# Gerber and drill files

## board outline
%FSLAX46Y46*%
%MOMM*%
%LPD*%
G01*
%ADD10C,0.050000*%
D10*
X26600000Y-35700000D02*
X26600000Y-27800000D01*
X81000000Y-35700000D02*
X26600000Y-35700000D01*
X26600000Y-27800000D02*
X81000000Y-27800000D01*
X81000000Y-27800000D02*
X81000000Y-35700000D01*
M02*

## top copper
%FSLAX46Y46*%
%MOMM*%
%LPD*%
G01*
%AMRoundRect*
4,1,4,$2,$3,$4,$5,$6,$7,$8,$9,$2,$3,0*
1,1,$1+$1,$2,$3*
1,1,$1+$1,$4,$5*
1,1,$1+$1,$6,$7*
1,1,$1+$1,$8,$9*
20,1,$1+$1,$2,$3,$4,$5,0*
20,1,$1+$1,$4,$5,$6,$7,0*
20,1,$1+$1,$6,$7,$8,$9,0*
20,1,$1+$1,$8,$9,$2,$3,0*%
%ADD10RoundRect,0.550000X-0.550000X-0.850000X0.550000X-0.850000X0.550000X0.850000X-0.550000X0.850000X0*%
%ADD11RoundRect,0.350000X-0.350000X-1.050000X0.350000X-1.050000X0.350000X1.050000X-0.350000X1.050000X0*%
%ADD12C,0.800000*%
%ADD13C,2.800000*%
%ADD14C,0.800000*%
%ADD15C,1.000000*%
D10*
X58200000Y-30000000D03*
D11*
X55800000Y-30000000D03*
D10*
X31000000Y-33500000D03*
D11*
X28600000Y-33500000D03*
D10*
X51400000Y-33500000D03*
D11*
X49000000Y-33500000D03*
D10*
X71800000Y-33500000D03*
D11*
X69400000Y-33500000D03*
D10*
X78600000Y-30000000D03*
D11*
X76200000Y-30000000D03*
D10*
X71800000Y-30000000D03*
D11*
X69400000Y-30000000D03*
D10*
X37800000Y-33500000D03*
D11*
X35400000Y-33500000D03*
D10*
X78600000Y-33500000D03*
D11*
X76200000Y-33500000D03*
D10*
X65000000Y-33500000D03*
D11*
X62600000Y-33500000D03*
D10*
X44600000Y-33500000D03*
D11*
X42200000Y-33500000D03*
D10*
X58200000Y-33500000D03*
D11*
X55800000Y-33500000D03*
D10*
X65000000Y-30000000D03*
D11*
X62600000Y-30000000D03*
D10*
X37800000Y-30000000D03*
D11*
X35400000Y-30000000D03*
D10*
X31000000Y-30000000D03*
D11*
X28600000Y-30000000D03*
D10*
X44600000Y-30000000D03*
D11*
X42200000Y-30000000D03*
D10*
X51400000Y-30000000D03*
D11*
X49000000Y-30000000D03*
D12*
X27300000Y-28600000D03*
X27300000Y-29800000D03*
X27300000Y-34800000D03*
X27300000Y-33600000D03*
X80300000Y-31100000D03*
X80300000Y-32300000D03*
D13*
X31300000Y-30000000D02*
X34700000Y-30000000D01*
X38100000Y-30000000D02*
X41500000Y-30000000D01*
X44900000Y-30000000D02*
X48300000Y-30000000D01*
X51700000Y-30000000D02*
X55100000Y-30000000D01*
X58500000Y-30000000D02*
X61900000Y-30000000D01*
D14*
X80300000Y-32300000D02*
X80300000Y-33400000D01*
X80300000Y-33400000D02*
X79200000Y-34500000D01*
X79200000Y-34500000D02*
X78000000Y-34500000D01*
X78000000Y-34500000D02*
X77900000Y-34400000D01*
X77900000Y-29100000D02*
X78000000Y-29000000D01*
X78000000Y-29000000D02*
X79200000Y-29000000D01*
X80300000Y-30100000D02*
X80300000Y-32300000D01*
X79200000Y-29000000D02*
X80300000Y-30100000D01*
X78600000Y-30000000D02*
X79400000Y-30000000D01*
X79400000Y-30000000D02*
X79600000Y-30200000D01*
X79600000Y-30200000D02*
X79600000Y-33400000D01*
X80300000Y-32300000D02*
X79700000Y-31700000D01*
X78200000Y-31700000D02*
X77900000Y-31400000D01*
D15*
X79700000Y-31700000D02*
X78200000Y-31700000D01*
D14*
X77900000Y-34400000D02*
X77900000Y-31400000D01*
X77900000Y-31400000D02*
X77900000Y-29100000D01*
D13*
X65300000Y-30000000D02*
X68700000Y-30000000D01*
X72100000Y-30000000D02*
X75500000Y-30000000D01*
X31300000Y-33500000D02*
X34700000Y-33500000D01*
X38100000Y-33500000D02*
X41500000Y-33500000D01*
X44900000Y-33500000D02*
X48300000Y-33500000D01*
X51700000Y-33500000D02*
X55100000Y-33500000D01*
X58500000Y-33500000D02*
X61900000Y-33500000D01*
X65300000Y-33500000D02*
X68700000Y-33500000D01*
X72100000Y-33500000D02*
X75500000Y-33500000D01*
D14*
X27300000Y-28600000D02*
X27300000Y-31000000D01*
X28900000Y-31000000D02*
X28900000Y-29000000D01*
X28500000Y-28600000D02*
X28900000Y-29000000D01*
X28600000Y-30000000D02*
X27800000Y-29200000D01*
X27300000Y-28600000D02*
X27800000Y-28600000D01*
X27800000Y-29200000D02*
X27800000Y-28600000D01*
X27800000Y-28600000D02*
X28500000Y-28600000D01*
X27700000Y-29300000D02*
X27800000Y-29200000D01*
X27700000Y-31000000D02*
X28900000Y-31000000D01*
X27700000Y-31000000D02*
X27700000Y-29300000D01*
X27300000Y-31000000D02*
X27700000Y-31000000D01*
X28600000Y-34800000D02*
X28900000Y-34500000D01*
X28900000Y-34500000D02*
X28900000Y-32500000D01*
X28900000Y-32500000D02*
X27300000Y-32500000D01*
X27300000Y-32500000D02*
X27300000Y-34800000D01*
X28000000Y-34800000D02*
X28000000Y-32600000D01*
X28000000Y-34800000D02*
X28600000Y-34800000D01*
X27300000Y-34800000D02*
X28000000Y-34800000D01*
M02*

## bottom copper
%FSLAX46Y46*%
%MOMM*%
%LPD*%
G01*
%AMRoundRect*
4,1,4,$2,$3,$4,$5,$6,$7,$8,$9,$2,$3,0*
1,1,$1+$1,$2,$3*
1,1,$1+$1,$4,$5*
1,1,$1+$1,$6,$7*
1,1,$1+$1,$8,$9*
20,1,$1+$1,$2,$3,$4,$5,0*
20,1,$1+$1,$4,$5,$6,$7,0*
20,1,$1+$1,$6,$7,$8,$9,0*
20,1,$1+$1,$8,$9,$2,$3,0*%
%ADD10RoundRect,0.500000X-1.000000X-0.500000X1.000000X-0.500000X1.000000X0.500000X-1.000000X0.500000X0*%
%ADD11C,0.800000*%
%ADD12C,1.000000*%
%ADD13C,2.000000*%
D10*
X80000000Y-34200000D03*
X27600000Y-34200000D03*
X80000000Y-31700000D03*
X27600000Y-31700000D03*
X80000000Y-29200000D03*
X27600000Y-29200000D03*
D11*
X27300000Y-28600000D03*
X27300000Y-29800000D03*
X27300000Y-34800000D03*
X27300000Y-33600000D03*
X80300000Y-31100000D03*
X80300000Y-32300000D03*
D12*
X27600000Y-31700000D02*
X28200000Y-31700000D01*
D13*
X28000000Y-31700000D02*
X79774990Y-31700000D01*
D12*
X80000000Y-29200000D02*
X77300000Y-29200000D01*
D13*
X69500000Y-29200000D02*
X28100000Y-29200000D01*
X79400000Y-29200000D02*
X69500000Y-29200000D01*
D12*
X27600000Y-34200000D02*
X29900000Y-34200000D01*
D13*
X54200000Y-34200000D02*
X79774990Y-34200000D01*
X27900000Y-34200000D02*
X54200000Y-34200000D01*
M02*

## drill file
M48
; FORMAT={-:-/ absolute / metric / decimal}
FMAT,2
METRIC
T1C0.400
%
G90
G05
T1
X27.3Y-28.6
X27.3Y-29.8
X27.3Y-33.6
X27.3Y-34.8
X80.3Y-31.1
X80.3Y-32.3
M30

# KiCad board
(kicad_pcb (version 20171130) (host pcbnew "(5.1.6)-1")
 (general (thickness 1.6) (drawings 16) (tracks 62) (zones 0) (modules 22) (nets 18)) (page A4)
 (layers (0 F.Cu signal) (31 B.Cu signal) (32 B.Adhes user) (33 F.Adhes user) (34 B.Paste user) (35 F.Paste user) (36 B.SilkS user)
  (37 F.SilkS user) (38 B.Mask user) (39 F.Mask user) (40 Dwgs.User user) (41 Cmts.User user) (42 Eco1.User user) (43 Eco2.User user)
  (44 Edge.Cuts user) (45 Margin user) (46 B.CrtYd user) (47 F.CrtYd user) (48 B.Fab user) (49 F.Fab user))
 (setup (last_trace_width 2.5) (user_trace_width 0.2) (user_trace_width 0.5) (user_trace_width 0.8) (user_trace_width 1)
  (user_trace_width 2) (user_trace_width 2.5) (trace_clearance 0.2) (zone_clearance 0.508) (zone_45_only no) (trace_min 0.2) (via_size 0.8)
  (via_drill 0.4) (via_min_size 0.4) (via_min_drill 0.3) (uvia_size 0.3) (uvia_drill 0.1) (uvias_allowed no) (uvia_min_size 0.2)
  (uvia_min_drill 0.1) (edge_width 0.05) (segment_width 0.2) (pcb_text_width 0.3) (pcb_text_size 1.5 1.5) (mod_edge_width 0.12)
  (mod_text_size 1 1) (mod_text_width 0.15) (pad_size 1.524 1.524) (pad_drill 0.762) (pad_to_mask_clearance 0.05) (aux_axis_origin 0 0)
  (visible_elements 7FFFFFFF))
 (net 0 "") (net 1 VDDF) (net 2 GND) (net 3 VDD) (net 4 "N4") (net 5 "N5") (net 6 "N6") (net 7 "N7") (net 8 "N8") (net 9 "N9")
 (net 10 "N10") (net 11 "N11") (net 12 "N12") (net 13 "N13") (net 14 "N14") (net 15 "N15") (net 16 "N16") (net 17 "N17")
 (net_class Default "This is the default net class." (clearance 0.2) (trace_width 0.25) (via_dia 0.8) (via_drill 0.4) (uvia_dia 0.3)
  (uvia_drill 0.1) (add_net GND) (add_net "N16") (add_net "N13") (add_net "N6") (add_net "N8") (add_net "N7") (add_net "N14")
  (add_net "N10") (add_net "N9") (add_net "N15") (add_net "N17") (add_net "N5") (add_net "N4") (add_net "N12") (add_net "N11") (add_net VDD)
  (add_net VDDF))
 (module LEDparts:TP (layer B.Cu) (at 80 34.2)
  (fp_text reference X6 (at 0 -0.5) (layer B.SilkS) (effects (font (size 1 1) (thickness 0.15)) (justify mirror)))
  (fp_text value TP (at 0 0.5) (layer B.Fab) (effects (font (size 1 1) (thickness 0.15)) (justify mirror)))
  (pad 1 smd roundrect (at 0 0) (size 3 2) (layers B.Cu B.Paste B.Mask) (roundrect_rratio 0.25) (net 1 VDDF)))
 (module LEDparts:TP (layer B.Cu) (at 27.6 34.2)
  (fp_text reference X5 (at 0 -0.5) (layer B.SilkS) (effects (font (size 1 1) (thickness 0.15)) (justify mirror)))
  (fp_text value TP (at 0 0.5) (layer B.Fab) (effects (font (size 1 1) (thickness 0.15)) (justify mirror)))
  (pad 1 smd roundrect (at 0 0) (size 3 2) (layers B.Cu B.Paste B.Mask) (roundrect_rratio 0.25) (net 1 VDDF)))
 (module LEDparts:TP (layer B.Cu) (at 80 31.7)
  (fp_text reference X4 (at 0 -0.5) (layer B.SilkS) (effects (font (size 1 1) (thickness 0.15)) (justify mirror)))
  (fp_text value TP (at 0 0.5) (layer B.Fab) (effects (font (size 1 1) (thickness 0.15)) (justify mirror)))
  (pad 1 smd roundrect (at 0 0) (size 3 2) (layers B.Cu B.Paste B.Mask) (roundrect_rratio 0.25) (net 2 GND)))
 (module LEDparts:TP (layer B.Cu) (at 27.6 31.7)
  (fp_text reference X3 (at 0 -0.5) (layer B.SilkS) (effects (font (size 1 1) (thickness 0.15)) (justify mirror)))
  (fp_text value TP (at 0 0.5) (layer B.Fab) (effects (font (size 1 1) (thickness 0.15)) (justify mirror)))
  (pad 1 smd roundrect (at 0 0) (size 3 2) (layers B.Cu B.Paste B.Mask) (roundrect_rratio 0.25) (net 2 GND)))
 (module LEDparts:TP (layer B.Cu) (at 80 29.2)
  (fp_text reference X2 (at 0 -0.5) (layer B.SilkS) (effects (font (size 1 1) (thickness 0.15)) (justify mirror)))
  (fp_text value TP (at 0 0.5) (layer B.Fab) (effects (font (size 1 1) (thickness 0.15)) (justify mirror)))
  (pad 1 smd roundrect (at 0 0) (size 3 2) (layers B.Cu B.Paste B.Mask) (roundrect_rratio 0.25) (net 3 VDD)))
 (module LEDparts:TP (layer B.Cu) (at 27.6 29.2)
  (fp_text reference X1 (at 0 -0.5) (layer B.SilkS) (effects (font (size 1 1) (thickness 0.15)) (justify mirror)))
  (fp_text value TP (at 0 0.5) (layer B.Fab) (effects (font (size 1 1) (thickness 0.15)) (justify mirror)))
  (pad 1 smd roundrect (at 0 0) (size 3 2) (layers B.Cu B.Paste B.Mask) (roundrect_rratio 0.25) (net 3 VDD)))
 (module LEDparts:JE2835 (layer F.Cu) (at 57.2 30)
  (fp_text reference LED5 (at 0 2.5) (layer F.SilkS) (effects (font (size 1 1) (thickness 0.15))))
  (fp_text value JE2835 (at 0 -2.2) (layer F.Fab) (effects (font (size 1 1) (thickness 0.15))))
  (pad 1 smd roundrect (at 1 0) (size 2.2 2.8) (layers F.Cu F.Paste F.Mask) (roundrect_rratio 0.25) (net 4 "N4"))
  (pad 2 smd roundrect (at -1.4 0) (size 1.4 2.8) (layers F.Cu F.Paste F.Mask) (roundrect_rratio 0.25) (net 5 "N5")))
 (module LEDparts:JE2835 (layer F.Cu) (at 30 33.5)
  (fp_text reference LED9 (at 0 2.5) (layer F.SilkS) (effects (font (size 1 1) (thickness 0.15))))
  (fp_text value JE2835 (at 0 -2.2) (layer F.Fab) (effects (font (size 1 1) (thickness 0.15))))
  (pad 1 smd roundrect (at 1 0) (size 2.2 2.8) (layers F.Cu F.Paste F.Mask) (roundrect_rratio 0.25) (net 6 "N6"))
  (pad 2 smd roundrect (at -1.4 0) (size 1.4 2.8) (layers F.Cu F.Paste F.Mask) (roundrect_rratio 0.25) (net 1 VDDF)))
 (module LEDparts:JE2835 (layer F.Cu) (at 50.4 33.5)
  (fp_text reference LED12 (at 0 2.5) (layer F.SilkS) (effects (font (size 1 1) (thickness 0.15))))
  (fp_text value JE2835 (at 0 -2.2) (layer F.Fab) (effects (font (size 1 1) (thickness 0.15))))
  (pad 1 smd roundrect (at 1 0) (size 2.2 2.8) (layers F.Cu F.Paste F.Mask) (roundrect_rratio 0.25) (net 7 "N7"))
  (pad 2 smd roundrect (at -1.4 0) (size 1.4 2.8) (layers F.Cu F.Paste F.Mask) (roundrect_rratio 0.25) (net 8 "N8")))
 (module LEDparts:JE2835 (layer F.Cu) (at 70.8 33.5)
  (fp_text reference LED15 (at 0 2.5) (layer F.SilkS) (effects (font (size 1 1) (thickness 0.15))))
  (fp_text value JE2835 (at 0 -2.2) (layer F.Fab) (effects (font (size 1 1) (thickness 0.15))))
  (pad 1 smd roundrect (at 1 0) (size 2.2 2.8) (layers F.Cu F.Paste F.Mask) (roundrect_rratio 0.25) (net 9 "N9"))
  (pad 2 smd roundrect (at -1.4 0) (size 1.4 2.8) (layers F.Cu F.Paste F.Mask) (roundrect_rratio 0.25) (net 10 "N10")))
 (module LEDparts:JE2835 (layer F.Cu) (at 77.6 30)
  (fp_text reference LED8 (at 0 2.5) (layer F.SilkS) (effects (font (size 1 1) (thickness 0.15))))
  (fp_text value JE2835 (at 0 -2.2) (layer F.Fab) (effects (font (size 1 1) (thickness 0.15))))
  (pad 1 smd roundrect (at 1 0) (size 2.2 2.8) (layers F.Cu F.Paste F.Mask) (roundrect_rratio 0.25) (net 2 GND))
  (pad 2 smd roundrect (at -1.4 0) (size 1.4 2.8) (layers F.Cu F.Paste F.Mask) (roundrect_rratio 0.25) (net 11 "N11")))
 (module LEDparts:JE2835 (layer F.Cu) (at 70.8 30)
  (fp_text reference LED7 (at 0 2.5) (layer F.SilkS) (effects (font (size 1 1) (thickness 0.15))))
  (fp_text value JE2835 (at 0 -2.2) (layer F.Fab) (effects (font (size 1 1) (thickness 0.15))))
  (pad 1 smd roundrect (at 1 0) (size 2.2 2.8) (layers F.Cu F.Paste F.Mask) (roundrect_rratio 0.25) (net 11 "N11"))
  (pad 2 smd roundrect (at -1.4 0) (size 1.4 2.8) (layers F.Cu F.Paste F.Mask) (roundrect_rratio 0.25) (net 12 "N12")))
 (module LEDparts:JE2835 (layer F.Cu) (at 36.8 33.5)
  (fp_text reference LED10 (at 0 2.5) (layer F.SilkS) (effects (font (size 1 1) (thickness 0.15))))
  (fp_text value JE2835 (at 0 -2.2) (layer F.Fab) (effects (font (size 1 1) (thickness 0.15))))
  (pad 1 smd roundrect (at 1 0) (size 2.2 2.8) (layers F.Cu F.Paste F.Mask) (roundrect_rratio 0.25) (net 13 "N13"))
  (pad 2 smd roundrect (at -1.4 0) (size 1.4 2.8) (layers F.Cu F.Paste F.Mask) (roundrect_rratio 0.25) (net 6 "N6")))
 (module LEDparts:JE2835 (layer F.Cu) (at 77.6 33.5)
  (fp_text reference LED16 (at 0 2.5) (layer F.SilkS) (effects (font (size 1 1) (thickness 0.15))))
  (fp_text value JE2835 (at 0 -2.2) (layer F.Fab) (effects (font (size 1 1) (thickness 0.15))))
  (pad 1 smd roundrect (at 1 0) (size 2.2 2.8) (layers F.Cu F.Paste F.Mask) (roundrect_rratio 0.25) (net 2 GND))
  (pad 2 smd roundrect (at -1.4 0) (size 1.4 2.8) (layers F.Cu F.Paste F.Mask) (roundrect_rratio 0.25) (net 9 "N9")))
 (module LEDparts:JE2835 (layer F.Cu) (at 64 33.5)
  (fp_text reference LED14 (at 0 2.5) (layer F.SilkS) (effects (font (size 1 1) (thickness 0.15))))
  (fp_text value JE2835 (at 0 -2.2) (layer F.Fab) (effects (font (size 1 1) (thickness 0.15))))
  (pad 1 smd roundrect (at 1 0) (size 2.2 2.8) (layers F.Cu F.Paste F.Mask) (roundrect_rratio 0.25) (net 10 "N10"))
  (pad 2 smd roundrect (at -1.4 0) (size 1.4 2.8) (layers F.Cu F.Paste F.Mask) (roundrect_rratio 0.25) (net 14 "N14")))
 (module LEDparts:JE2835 (layer F.Cu) (at 43.6 33.5)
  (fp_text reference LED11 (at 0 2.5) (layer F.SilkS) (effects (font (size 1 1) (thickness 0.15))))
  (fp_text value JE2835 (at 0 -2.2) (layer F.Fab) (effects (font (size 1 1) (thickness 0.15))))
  (pad 1 smd roundrect (at 1 0) (size 2.2 2.8) (layers F.Cu F.Paste F.Mask) (roundrect_rratio 0.25) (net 8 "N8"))
  (pad 2 smd roundrect (at -1.4 0) (size 1.4 2.8) (layers F.Cu F.Paste F.Mask) (roundrect_rratio 0.25) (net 13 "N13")))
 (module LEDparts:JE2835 (layer F.Cu) (at 57.2 33.5)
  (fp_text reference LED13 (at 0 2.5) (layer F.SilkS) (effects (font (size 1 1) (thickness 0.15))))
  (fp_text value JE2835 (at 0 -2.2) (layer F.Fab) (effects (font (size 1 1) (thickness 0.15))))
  (pad 1 smd roundrect (at 1 0) (size 2.2 2.8) (layers F.Cu F.Paste F.Mask) (roundrect_rratio 0.25) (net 14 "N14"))
  (pad 2 smd roundrect (at -1.4 0) (size 1.4 2.8) (layers F.Cu F.Paste F.Mask) (roundrect_rratio 0.25) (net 7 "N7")))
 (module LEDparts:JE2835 (layer F.Cu) (at 64 30)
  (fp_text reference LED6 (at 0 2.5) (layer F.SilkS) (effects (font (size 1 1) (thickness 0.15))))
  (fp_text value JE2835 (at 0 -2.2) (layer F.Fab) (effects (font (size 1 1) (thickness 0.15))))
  (pad 1 smd roundrect (at 1 0) (size 2.2 2.8) (layers F.Cu F.Paste F.Mask) (roundrect_rratio 0.25) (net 12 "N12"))
  (pad 2 smd roundrect (at -1.4 0) (size 1.4 2.8) (layers F.Cu F.Paste F.Mask) (roundrect_rratio 0.25) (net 4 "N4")))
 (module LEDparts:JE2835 (layer F.Cu) (at 36.8 30)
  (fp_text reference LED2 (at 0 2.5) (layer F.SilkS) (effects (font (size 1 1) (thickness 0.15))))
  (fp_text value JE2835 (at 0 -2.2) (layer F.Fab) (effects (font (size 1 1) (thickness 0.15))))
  (pad 1 smd roundrect (at 1 0) (size 2.2 2.8) (layers F.Cu F.Paste F.Mask) (roundrect_rratio 0.25) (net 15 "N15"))
  (pad 2 smd roundrect (at -1.4 0) (size 1.4 2.8) (layers F.Cu F.Paste F.Mask) (roundrect_rratio 0.25) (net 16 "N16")))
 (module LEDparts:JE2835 (layer F.Cu) (at 30 30)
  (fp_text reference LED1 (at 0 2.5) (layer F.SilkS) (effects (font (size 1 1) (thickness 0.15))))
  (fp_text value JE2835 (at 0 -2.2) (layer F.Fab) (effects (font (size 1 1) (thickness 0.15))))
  (pad 1 smd roundrect (at 1 0) (size 2.2 2.8) (layers F.Cu F.Paste F.Mask) (roundrect_rratio 0.25) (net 16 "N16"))
  (pad 2 smd roundrect (at -1.4 0) (size 1.4 2.8) (layers F.Cu F.Paste F.Mask) (roundrect_rratio 0.25) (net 3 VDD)))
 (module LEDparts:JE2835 (layer F.Cu) (at 43.6 30)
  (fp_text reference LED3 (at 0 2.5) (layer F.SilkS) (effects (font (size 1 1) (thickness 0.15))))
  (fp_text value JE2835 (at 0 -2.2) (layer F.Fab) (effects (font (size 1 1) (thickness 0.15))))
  (pad 1 smd roundrect (at 1 0) (size 2.2 2.8) (layers F.Cu F.Paste F.Mask) (roundrect_rratio 0.25) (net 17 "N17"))
  (pad 2 smd roundrect (at -1.4 0) (size 1.4 2.8) (layers F.Cu F.Paste F.Mask) (roundrect_rratio 0.25) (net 15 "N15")))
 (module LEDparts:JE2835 (layer F.Cu) (at 50.4 30)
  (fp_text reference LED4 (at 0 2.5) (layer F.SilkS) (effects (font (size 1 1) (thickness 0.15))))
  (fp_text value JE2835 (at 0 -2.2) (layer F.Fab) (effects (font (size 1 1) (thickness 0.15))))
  (pad 1 smd roundrect (at 1 0) (size 2.2 2.8) (layers F.Cu F.Paste F.Mask) (roundrect_rratio 0.25) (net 5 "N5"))
  (pad 2 smd roundrect (at -1.4 0) (size 1.4 2.8) (layers F.Cu F.Paste F.Mask) (roundrect_rratio 0.25) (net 17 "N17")))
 (gr_line (start 26.6 35.7) (end 26.6 27.8) (layer Edge.Cuts) (width 0.05))
 (gr_line (start 81 35.7) (end 26.6 35.7) (layer Edge.Cuts) (width 0.05))
 (gr_line (start 26.6 27.8) (end 81 27.8) (layer Edge.Cuts) (width 0.05))
 (gr_line (start 81 27.8) (end 81 35.7) (layer Edge.Cuts) (width 0.05))
 (segment (start 31.3 30) (end 34.7 30) (width 2.8) (layer F.Cu) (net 16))
 (segment (start 38.1 30) (end 41.5 30) (width 2.8) (layer F.Cu) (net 15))
 (segment (start 44.9 30) (end 48.3 30) (width 2.8) (layer F.Cu) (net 17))
 (segment (start 51.7 30) (end 55.1 30) (width 2.8) (layer F.Cu) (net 5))
 (segment (start 58.5 30) (end 61.9 30) (width 2.8) (layer F.Cu) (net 4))
 (via (at 27.3 28.6) (size 0.8) (drill 0.4) (layers F.Cu B.Cu) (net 3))
 (via (at 27.3 29.8) (size 0.8) (drill 0.4) (layers F.Cu B.Cu) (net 3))
 (via (at 27.3 34.8) (size 0.8) (drill 0.4) (layers F.Cu B.Cu) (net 1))
 (via (at 27.3 33.6) (size 0.8) (drill 0.4) (layers F.Cu B.Cu) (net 1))
 (via (at 80.3 31.1) (size 0.8) (drill 0.4) (layers F.Cu B.Cu) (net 2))
 (via (at 80.3 32.3) (size 0.8) (drill 0.4) (layers F.Cu B.Cu) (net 2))
 (segment (start 27.6 31.7) (end 28.2 31.7) (width 1) (layer B.Cu) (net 2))
 (segment (start 28 31.7) (end 79.77499 31.7) (width 2) (layer B.Cu) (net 2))
 (segment (start 80.3 32.3) (end 80.3 33.4) (width 0.8) (layer F.Cu) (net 2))
 (segment (start 80.3 33.4) (end 79.2 34.5) (width 0.8) (layer F.Cu) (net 2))
 (segment (start 79.2 34.5) (end 78 34.5) (width 0.8) (layer F.Cu) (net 2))
 (segment (start 78 34.5) (end 77.9 34.4) (width 0.8) (layer F.Cu) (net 2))
 (segment (start 77.9 29.1) (end 78 29) (width 0.8) (layer F.Cu) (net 2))
 (segment (start 78 29) (end 79.2 29) (width 0.8) (layer F.Cu) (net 2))
 (segment (start 80.3 30.1) (end 80.3 32.3) (width 0.8) (layer F.Cu) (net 2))
 (segment (start 79.2 29) (end 80.3 30.1) (width 0.8) (layer F.Cu) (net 2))
 (segment (start 78.6 30) (end 79.4 30) (width 0.8) (layer F.Cu) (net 2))
 (segment (start 79.4 30) (end 79.6 30.2) (width 0.8) (layer F.Cu) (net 2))
 (segment (start 79.6 30.2) (end 79.6 33.4) (width 0.8) (layer F.Cu) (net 2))
 (segment (start 80.3 32.3) (end 79.7 31.7) (width 0.8) (layer F.Cu) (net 2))
 (segment (start 78.2 31.7) (end 77.9 31.4) (width 0.8) (layer F.Cu) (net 2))
 (segment (start 79.7 31.7) (end 78.2 31.7) (width 1) (layer F.Cu) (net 2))
 (segment (start 77.9 34.4) (end 77.9 31.4) (width 0.8) (layer F.Cu) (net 2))
 (segment (start 77.9 31.4) (end 77.9 29.1) (width 0.8) (layer F.Cu) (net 2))
 (segment (start 65.3 30) (end 68.7 30) (width 2.8) (layer F.Cu) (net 12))
 (segment (start 72.1 30) (end 75.5 30) (width 2.8) (layer F.Cu) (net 11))
 (segment (start 31.3 33.5) (end 34.7 33.5) (width 2.8) (layer F.Cu) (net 6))
 (segment (start 38.1 33.5) (end 41.5 33.5) (width 2.8) (layer F.Cu) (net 13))
 (segment (start 44.9 33.5) (end 48.3 33.5) (width 2.8) (layer F.Cu) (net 8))
 (segment (start 51.7 33.5) (end 55.1 33.5) (width 2.8) (layer F.Cu) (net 7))
 (segment (start 58.5 33.5) (end 61.9 33.5) (width 2.8) (layer F.Cu) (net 14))
 (segment (start 65.3 33.5) (end 68.7 33.5) (width 2.8) (layer F.Cu) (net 10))
 (segment (start 72.1 33.5) (end 75.5 33.5) (width 2.8) (layer F.Cu) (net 9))
 (segment (start 80 29.2) (end 77.3 29.2) (width 1) (layer B.Cu) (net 3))
 (segment (start 69.5 29.2) (end 28.1 29.2) (width 2) (layer B.Cu) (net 3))
 (segment (start 79.4 29.2) (end 69.5 29.2) (width 2) (layer B.Cu) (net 3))
 (segment (start 27.3 28.6) (end 27.3 31) (width 0.8) (layer F.Cu) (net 3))
 (segment (start 28.9 31) (end 28.9 29) (width 0.8) (layer F.Cu) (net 3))
 (segment (start 28.5 28.6) (end 28.9 29) (width 0.8) (layer F.Cu) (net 3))
 (segment (start 28.6 30) (end 27.8 29.2) (width 0.8) (layer F.Cu) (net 3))
 (segment (start 27.3 28.6) (end 27.8 28.6) (width 0.8) (layer F.Cu) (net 3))
 (segment (start 27.8 29.2) (end 27.8 28.6) (width 0.8) (layer F.Cu) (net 3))
 (segment (start 27.8 28.6) (end 28.5 28.6) (width 0.8) (layer F.Cu) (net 3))
 (segment (start 27.7 29.3) (end 27.8 29.2) (width 0.8) (layer F.Cu) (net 3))
 (segment (start 27.7 31) (end 28.9 31) (width 0.8) (layer F.Cu) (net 3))
 (segment (start 27.7 31) (end 27.7 29.3) (width 0.8) (layer F.Cu) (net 3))
 (segment (start 27.3 31) (end 27.7 31) (width 0.8) (layer F.Cu) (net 3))
 (segment (start 27.6 34.2) (end 29.9 34.2) (width 1) (layer B.Cu) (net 1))
 (segment (start 54.2 34.2) (end 79.77499 34.2) (width 2) (layer B.Cu) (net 1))
 (segment (start 27.9 34.2) (end 54.2 34.2) (width 2) (layer B.Cu) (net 1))
 (segment (start 28.6 34.8) (end 28.9 34.5) (width 0.8) (layer F.Cu) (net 1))
 (segment (start 28.9 34.5) (end 28.9 32.5) (width 0.8) (layer F.Cu) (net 1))
 (segment (start 28.9 32.5) (end 27.3 32.5) (width 0.8) (layer F.Cu) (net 1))
 (segment (start 27.3 32.5) (end 27.3 34.8) (width 0.8) (layer F.Cu) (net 1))
 (segment (start 28 34.8) (end 28 32.6) (width 0.8) (layer F.Cu) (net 1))
 (segment (start 28 34.8) (end 28.6 34.8) (width 0.8) (layer F.Cu) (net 1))
 (segment (start 27.3 34.8) (end 28 34.8) (width 0.8) (layer F.Cu) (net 1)))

